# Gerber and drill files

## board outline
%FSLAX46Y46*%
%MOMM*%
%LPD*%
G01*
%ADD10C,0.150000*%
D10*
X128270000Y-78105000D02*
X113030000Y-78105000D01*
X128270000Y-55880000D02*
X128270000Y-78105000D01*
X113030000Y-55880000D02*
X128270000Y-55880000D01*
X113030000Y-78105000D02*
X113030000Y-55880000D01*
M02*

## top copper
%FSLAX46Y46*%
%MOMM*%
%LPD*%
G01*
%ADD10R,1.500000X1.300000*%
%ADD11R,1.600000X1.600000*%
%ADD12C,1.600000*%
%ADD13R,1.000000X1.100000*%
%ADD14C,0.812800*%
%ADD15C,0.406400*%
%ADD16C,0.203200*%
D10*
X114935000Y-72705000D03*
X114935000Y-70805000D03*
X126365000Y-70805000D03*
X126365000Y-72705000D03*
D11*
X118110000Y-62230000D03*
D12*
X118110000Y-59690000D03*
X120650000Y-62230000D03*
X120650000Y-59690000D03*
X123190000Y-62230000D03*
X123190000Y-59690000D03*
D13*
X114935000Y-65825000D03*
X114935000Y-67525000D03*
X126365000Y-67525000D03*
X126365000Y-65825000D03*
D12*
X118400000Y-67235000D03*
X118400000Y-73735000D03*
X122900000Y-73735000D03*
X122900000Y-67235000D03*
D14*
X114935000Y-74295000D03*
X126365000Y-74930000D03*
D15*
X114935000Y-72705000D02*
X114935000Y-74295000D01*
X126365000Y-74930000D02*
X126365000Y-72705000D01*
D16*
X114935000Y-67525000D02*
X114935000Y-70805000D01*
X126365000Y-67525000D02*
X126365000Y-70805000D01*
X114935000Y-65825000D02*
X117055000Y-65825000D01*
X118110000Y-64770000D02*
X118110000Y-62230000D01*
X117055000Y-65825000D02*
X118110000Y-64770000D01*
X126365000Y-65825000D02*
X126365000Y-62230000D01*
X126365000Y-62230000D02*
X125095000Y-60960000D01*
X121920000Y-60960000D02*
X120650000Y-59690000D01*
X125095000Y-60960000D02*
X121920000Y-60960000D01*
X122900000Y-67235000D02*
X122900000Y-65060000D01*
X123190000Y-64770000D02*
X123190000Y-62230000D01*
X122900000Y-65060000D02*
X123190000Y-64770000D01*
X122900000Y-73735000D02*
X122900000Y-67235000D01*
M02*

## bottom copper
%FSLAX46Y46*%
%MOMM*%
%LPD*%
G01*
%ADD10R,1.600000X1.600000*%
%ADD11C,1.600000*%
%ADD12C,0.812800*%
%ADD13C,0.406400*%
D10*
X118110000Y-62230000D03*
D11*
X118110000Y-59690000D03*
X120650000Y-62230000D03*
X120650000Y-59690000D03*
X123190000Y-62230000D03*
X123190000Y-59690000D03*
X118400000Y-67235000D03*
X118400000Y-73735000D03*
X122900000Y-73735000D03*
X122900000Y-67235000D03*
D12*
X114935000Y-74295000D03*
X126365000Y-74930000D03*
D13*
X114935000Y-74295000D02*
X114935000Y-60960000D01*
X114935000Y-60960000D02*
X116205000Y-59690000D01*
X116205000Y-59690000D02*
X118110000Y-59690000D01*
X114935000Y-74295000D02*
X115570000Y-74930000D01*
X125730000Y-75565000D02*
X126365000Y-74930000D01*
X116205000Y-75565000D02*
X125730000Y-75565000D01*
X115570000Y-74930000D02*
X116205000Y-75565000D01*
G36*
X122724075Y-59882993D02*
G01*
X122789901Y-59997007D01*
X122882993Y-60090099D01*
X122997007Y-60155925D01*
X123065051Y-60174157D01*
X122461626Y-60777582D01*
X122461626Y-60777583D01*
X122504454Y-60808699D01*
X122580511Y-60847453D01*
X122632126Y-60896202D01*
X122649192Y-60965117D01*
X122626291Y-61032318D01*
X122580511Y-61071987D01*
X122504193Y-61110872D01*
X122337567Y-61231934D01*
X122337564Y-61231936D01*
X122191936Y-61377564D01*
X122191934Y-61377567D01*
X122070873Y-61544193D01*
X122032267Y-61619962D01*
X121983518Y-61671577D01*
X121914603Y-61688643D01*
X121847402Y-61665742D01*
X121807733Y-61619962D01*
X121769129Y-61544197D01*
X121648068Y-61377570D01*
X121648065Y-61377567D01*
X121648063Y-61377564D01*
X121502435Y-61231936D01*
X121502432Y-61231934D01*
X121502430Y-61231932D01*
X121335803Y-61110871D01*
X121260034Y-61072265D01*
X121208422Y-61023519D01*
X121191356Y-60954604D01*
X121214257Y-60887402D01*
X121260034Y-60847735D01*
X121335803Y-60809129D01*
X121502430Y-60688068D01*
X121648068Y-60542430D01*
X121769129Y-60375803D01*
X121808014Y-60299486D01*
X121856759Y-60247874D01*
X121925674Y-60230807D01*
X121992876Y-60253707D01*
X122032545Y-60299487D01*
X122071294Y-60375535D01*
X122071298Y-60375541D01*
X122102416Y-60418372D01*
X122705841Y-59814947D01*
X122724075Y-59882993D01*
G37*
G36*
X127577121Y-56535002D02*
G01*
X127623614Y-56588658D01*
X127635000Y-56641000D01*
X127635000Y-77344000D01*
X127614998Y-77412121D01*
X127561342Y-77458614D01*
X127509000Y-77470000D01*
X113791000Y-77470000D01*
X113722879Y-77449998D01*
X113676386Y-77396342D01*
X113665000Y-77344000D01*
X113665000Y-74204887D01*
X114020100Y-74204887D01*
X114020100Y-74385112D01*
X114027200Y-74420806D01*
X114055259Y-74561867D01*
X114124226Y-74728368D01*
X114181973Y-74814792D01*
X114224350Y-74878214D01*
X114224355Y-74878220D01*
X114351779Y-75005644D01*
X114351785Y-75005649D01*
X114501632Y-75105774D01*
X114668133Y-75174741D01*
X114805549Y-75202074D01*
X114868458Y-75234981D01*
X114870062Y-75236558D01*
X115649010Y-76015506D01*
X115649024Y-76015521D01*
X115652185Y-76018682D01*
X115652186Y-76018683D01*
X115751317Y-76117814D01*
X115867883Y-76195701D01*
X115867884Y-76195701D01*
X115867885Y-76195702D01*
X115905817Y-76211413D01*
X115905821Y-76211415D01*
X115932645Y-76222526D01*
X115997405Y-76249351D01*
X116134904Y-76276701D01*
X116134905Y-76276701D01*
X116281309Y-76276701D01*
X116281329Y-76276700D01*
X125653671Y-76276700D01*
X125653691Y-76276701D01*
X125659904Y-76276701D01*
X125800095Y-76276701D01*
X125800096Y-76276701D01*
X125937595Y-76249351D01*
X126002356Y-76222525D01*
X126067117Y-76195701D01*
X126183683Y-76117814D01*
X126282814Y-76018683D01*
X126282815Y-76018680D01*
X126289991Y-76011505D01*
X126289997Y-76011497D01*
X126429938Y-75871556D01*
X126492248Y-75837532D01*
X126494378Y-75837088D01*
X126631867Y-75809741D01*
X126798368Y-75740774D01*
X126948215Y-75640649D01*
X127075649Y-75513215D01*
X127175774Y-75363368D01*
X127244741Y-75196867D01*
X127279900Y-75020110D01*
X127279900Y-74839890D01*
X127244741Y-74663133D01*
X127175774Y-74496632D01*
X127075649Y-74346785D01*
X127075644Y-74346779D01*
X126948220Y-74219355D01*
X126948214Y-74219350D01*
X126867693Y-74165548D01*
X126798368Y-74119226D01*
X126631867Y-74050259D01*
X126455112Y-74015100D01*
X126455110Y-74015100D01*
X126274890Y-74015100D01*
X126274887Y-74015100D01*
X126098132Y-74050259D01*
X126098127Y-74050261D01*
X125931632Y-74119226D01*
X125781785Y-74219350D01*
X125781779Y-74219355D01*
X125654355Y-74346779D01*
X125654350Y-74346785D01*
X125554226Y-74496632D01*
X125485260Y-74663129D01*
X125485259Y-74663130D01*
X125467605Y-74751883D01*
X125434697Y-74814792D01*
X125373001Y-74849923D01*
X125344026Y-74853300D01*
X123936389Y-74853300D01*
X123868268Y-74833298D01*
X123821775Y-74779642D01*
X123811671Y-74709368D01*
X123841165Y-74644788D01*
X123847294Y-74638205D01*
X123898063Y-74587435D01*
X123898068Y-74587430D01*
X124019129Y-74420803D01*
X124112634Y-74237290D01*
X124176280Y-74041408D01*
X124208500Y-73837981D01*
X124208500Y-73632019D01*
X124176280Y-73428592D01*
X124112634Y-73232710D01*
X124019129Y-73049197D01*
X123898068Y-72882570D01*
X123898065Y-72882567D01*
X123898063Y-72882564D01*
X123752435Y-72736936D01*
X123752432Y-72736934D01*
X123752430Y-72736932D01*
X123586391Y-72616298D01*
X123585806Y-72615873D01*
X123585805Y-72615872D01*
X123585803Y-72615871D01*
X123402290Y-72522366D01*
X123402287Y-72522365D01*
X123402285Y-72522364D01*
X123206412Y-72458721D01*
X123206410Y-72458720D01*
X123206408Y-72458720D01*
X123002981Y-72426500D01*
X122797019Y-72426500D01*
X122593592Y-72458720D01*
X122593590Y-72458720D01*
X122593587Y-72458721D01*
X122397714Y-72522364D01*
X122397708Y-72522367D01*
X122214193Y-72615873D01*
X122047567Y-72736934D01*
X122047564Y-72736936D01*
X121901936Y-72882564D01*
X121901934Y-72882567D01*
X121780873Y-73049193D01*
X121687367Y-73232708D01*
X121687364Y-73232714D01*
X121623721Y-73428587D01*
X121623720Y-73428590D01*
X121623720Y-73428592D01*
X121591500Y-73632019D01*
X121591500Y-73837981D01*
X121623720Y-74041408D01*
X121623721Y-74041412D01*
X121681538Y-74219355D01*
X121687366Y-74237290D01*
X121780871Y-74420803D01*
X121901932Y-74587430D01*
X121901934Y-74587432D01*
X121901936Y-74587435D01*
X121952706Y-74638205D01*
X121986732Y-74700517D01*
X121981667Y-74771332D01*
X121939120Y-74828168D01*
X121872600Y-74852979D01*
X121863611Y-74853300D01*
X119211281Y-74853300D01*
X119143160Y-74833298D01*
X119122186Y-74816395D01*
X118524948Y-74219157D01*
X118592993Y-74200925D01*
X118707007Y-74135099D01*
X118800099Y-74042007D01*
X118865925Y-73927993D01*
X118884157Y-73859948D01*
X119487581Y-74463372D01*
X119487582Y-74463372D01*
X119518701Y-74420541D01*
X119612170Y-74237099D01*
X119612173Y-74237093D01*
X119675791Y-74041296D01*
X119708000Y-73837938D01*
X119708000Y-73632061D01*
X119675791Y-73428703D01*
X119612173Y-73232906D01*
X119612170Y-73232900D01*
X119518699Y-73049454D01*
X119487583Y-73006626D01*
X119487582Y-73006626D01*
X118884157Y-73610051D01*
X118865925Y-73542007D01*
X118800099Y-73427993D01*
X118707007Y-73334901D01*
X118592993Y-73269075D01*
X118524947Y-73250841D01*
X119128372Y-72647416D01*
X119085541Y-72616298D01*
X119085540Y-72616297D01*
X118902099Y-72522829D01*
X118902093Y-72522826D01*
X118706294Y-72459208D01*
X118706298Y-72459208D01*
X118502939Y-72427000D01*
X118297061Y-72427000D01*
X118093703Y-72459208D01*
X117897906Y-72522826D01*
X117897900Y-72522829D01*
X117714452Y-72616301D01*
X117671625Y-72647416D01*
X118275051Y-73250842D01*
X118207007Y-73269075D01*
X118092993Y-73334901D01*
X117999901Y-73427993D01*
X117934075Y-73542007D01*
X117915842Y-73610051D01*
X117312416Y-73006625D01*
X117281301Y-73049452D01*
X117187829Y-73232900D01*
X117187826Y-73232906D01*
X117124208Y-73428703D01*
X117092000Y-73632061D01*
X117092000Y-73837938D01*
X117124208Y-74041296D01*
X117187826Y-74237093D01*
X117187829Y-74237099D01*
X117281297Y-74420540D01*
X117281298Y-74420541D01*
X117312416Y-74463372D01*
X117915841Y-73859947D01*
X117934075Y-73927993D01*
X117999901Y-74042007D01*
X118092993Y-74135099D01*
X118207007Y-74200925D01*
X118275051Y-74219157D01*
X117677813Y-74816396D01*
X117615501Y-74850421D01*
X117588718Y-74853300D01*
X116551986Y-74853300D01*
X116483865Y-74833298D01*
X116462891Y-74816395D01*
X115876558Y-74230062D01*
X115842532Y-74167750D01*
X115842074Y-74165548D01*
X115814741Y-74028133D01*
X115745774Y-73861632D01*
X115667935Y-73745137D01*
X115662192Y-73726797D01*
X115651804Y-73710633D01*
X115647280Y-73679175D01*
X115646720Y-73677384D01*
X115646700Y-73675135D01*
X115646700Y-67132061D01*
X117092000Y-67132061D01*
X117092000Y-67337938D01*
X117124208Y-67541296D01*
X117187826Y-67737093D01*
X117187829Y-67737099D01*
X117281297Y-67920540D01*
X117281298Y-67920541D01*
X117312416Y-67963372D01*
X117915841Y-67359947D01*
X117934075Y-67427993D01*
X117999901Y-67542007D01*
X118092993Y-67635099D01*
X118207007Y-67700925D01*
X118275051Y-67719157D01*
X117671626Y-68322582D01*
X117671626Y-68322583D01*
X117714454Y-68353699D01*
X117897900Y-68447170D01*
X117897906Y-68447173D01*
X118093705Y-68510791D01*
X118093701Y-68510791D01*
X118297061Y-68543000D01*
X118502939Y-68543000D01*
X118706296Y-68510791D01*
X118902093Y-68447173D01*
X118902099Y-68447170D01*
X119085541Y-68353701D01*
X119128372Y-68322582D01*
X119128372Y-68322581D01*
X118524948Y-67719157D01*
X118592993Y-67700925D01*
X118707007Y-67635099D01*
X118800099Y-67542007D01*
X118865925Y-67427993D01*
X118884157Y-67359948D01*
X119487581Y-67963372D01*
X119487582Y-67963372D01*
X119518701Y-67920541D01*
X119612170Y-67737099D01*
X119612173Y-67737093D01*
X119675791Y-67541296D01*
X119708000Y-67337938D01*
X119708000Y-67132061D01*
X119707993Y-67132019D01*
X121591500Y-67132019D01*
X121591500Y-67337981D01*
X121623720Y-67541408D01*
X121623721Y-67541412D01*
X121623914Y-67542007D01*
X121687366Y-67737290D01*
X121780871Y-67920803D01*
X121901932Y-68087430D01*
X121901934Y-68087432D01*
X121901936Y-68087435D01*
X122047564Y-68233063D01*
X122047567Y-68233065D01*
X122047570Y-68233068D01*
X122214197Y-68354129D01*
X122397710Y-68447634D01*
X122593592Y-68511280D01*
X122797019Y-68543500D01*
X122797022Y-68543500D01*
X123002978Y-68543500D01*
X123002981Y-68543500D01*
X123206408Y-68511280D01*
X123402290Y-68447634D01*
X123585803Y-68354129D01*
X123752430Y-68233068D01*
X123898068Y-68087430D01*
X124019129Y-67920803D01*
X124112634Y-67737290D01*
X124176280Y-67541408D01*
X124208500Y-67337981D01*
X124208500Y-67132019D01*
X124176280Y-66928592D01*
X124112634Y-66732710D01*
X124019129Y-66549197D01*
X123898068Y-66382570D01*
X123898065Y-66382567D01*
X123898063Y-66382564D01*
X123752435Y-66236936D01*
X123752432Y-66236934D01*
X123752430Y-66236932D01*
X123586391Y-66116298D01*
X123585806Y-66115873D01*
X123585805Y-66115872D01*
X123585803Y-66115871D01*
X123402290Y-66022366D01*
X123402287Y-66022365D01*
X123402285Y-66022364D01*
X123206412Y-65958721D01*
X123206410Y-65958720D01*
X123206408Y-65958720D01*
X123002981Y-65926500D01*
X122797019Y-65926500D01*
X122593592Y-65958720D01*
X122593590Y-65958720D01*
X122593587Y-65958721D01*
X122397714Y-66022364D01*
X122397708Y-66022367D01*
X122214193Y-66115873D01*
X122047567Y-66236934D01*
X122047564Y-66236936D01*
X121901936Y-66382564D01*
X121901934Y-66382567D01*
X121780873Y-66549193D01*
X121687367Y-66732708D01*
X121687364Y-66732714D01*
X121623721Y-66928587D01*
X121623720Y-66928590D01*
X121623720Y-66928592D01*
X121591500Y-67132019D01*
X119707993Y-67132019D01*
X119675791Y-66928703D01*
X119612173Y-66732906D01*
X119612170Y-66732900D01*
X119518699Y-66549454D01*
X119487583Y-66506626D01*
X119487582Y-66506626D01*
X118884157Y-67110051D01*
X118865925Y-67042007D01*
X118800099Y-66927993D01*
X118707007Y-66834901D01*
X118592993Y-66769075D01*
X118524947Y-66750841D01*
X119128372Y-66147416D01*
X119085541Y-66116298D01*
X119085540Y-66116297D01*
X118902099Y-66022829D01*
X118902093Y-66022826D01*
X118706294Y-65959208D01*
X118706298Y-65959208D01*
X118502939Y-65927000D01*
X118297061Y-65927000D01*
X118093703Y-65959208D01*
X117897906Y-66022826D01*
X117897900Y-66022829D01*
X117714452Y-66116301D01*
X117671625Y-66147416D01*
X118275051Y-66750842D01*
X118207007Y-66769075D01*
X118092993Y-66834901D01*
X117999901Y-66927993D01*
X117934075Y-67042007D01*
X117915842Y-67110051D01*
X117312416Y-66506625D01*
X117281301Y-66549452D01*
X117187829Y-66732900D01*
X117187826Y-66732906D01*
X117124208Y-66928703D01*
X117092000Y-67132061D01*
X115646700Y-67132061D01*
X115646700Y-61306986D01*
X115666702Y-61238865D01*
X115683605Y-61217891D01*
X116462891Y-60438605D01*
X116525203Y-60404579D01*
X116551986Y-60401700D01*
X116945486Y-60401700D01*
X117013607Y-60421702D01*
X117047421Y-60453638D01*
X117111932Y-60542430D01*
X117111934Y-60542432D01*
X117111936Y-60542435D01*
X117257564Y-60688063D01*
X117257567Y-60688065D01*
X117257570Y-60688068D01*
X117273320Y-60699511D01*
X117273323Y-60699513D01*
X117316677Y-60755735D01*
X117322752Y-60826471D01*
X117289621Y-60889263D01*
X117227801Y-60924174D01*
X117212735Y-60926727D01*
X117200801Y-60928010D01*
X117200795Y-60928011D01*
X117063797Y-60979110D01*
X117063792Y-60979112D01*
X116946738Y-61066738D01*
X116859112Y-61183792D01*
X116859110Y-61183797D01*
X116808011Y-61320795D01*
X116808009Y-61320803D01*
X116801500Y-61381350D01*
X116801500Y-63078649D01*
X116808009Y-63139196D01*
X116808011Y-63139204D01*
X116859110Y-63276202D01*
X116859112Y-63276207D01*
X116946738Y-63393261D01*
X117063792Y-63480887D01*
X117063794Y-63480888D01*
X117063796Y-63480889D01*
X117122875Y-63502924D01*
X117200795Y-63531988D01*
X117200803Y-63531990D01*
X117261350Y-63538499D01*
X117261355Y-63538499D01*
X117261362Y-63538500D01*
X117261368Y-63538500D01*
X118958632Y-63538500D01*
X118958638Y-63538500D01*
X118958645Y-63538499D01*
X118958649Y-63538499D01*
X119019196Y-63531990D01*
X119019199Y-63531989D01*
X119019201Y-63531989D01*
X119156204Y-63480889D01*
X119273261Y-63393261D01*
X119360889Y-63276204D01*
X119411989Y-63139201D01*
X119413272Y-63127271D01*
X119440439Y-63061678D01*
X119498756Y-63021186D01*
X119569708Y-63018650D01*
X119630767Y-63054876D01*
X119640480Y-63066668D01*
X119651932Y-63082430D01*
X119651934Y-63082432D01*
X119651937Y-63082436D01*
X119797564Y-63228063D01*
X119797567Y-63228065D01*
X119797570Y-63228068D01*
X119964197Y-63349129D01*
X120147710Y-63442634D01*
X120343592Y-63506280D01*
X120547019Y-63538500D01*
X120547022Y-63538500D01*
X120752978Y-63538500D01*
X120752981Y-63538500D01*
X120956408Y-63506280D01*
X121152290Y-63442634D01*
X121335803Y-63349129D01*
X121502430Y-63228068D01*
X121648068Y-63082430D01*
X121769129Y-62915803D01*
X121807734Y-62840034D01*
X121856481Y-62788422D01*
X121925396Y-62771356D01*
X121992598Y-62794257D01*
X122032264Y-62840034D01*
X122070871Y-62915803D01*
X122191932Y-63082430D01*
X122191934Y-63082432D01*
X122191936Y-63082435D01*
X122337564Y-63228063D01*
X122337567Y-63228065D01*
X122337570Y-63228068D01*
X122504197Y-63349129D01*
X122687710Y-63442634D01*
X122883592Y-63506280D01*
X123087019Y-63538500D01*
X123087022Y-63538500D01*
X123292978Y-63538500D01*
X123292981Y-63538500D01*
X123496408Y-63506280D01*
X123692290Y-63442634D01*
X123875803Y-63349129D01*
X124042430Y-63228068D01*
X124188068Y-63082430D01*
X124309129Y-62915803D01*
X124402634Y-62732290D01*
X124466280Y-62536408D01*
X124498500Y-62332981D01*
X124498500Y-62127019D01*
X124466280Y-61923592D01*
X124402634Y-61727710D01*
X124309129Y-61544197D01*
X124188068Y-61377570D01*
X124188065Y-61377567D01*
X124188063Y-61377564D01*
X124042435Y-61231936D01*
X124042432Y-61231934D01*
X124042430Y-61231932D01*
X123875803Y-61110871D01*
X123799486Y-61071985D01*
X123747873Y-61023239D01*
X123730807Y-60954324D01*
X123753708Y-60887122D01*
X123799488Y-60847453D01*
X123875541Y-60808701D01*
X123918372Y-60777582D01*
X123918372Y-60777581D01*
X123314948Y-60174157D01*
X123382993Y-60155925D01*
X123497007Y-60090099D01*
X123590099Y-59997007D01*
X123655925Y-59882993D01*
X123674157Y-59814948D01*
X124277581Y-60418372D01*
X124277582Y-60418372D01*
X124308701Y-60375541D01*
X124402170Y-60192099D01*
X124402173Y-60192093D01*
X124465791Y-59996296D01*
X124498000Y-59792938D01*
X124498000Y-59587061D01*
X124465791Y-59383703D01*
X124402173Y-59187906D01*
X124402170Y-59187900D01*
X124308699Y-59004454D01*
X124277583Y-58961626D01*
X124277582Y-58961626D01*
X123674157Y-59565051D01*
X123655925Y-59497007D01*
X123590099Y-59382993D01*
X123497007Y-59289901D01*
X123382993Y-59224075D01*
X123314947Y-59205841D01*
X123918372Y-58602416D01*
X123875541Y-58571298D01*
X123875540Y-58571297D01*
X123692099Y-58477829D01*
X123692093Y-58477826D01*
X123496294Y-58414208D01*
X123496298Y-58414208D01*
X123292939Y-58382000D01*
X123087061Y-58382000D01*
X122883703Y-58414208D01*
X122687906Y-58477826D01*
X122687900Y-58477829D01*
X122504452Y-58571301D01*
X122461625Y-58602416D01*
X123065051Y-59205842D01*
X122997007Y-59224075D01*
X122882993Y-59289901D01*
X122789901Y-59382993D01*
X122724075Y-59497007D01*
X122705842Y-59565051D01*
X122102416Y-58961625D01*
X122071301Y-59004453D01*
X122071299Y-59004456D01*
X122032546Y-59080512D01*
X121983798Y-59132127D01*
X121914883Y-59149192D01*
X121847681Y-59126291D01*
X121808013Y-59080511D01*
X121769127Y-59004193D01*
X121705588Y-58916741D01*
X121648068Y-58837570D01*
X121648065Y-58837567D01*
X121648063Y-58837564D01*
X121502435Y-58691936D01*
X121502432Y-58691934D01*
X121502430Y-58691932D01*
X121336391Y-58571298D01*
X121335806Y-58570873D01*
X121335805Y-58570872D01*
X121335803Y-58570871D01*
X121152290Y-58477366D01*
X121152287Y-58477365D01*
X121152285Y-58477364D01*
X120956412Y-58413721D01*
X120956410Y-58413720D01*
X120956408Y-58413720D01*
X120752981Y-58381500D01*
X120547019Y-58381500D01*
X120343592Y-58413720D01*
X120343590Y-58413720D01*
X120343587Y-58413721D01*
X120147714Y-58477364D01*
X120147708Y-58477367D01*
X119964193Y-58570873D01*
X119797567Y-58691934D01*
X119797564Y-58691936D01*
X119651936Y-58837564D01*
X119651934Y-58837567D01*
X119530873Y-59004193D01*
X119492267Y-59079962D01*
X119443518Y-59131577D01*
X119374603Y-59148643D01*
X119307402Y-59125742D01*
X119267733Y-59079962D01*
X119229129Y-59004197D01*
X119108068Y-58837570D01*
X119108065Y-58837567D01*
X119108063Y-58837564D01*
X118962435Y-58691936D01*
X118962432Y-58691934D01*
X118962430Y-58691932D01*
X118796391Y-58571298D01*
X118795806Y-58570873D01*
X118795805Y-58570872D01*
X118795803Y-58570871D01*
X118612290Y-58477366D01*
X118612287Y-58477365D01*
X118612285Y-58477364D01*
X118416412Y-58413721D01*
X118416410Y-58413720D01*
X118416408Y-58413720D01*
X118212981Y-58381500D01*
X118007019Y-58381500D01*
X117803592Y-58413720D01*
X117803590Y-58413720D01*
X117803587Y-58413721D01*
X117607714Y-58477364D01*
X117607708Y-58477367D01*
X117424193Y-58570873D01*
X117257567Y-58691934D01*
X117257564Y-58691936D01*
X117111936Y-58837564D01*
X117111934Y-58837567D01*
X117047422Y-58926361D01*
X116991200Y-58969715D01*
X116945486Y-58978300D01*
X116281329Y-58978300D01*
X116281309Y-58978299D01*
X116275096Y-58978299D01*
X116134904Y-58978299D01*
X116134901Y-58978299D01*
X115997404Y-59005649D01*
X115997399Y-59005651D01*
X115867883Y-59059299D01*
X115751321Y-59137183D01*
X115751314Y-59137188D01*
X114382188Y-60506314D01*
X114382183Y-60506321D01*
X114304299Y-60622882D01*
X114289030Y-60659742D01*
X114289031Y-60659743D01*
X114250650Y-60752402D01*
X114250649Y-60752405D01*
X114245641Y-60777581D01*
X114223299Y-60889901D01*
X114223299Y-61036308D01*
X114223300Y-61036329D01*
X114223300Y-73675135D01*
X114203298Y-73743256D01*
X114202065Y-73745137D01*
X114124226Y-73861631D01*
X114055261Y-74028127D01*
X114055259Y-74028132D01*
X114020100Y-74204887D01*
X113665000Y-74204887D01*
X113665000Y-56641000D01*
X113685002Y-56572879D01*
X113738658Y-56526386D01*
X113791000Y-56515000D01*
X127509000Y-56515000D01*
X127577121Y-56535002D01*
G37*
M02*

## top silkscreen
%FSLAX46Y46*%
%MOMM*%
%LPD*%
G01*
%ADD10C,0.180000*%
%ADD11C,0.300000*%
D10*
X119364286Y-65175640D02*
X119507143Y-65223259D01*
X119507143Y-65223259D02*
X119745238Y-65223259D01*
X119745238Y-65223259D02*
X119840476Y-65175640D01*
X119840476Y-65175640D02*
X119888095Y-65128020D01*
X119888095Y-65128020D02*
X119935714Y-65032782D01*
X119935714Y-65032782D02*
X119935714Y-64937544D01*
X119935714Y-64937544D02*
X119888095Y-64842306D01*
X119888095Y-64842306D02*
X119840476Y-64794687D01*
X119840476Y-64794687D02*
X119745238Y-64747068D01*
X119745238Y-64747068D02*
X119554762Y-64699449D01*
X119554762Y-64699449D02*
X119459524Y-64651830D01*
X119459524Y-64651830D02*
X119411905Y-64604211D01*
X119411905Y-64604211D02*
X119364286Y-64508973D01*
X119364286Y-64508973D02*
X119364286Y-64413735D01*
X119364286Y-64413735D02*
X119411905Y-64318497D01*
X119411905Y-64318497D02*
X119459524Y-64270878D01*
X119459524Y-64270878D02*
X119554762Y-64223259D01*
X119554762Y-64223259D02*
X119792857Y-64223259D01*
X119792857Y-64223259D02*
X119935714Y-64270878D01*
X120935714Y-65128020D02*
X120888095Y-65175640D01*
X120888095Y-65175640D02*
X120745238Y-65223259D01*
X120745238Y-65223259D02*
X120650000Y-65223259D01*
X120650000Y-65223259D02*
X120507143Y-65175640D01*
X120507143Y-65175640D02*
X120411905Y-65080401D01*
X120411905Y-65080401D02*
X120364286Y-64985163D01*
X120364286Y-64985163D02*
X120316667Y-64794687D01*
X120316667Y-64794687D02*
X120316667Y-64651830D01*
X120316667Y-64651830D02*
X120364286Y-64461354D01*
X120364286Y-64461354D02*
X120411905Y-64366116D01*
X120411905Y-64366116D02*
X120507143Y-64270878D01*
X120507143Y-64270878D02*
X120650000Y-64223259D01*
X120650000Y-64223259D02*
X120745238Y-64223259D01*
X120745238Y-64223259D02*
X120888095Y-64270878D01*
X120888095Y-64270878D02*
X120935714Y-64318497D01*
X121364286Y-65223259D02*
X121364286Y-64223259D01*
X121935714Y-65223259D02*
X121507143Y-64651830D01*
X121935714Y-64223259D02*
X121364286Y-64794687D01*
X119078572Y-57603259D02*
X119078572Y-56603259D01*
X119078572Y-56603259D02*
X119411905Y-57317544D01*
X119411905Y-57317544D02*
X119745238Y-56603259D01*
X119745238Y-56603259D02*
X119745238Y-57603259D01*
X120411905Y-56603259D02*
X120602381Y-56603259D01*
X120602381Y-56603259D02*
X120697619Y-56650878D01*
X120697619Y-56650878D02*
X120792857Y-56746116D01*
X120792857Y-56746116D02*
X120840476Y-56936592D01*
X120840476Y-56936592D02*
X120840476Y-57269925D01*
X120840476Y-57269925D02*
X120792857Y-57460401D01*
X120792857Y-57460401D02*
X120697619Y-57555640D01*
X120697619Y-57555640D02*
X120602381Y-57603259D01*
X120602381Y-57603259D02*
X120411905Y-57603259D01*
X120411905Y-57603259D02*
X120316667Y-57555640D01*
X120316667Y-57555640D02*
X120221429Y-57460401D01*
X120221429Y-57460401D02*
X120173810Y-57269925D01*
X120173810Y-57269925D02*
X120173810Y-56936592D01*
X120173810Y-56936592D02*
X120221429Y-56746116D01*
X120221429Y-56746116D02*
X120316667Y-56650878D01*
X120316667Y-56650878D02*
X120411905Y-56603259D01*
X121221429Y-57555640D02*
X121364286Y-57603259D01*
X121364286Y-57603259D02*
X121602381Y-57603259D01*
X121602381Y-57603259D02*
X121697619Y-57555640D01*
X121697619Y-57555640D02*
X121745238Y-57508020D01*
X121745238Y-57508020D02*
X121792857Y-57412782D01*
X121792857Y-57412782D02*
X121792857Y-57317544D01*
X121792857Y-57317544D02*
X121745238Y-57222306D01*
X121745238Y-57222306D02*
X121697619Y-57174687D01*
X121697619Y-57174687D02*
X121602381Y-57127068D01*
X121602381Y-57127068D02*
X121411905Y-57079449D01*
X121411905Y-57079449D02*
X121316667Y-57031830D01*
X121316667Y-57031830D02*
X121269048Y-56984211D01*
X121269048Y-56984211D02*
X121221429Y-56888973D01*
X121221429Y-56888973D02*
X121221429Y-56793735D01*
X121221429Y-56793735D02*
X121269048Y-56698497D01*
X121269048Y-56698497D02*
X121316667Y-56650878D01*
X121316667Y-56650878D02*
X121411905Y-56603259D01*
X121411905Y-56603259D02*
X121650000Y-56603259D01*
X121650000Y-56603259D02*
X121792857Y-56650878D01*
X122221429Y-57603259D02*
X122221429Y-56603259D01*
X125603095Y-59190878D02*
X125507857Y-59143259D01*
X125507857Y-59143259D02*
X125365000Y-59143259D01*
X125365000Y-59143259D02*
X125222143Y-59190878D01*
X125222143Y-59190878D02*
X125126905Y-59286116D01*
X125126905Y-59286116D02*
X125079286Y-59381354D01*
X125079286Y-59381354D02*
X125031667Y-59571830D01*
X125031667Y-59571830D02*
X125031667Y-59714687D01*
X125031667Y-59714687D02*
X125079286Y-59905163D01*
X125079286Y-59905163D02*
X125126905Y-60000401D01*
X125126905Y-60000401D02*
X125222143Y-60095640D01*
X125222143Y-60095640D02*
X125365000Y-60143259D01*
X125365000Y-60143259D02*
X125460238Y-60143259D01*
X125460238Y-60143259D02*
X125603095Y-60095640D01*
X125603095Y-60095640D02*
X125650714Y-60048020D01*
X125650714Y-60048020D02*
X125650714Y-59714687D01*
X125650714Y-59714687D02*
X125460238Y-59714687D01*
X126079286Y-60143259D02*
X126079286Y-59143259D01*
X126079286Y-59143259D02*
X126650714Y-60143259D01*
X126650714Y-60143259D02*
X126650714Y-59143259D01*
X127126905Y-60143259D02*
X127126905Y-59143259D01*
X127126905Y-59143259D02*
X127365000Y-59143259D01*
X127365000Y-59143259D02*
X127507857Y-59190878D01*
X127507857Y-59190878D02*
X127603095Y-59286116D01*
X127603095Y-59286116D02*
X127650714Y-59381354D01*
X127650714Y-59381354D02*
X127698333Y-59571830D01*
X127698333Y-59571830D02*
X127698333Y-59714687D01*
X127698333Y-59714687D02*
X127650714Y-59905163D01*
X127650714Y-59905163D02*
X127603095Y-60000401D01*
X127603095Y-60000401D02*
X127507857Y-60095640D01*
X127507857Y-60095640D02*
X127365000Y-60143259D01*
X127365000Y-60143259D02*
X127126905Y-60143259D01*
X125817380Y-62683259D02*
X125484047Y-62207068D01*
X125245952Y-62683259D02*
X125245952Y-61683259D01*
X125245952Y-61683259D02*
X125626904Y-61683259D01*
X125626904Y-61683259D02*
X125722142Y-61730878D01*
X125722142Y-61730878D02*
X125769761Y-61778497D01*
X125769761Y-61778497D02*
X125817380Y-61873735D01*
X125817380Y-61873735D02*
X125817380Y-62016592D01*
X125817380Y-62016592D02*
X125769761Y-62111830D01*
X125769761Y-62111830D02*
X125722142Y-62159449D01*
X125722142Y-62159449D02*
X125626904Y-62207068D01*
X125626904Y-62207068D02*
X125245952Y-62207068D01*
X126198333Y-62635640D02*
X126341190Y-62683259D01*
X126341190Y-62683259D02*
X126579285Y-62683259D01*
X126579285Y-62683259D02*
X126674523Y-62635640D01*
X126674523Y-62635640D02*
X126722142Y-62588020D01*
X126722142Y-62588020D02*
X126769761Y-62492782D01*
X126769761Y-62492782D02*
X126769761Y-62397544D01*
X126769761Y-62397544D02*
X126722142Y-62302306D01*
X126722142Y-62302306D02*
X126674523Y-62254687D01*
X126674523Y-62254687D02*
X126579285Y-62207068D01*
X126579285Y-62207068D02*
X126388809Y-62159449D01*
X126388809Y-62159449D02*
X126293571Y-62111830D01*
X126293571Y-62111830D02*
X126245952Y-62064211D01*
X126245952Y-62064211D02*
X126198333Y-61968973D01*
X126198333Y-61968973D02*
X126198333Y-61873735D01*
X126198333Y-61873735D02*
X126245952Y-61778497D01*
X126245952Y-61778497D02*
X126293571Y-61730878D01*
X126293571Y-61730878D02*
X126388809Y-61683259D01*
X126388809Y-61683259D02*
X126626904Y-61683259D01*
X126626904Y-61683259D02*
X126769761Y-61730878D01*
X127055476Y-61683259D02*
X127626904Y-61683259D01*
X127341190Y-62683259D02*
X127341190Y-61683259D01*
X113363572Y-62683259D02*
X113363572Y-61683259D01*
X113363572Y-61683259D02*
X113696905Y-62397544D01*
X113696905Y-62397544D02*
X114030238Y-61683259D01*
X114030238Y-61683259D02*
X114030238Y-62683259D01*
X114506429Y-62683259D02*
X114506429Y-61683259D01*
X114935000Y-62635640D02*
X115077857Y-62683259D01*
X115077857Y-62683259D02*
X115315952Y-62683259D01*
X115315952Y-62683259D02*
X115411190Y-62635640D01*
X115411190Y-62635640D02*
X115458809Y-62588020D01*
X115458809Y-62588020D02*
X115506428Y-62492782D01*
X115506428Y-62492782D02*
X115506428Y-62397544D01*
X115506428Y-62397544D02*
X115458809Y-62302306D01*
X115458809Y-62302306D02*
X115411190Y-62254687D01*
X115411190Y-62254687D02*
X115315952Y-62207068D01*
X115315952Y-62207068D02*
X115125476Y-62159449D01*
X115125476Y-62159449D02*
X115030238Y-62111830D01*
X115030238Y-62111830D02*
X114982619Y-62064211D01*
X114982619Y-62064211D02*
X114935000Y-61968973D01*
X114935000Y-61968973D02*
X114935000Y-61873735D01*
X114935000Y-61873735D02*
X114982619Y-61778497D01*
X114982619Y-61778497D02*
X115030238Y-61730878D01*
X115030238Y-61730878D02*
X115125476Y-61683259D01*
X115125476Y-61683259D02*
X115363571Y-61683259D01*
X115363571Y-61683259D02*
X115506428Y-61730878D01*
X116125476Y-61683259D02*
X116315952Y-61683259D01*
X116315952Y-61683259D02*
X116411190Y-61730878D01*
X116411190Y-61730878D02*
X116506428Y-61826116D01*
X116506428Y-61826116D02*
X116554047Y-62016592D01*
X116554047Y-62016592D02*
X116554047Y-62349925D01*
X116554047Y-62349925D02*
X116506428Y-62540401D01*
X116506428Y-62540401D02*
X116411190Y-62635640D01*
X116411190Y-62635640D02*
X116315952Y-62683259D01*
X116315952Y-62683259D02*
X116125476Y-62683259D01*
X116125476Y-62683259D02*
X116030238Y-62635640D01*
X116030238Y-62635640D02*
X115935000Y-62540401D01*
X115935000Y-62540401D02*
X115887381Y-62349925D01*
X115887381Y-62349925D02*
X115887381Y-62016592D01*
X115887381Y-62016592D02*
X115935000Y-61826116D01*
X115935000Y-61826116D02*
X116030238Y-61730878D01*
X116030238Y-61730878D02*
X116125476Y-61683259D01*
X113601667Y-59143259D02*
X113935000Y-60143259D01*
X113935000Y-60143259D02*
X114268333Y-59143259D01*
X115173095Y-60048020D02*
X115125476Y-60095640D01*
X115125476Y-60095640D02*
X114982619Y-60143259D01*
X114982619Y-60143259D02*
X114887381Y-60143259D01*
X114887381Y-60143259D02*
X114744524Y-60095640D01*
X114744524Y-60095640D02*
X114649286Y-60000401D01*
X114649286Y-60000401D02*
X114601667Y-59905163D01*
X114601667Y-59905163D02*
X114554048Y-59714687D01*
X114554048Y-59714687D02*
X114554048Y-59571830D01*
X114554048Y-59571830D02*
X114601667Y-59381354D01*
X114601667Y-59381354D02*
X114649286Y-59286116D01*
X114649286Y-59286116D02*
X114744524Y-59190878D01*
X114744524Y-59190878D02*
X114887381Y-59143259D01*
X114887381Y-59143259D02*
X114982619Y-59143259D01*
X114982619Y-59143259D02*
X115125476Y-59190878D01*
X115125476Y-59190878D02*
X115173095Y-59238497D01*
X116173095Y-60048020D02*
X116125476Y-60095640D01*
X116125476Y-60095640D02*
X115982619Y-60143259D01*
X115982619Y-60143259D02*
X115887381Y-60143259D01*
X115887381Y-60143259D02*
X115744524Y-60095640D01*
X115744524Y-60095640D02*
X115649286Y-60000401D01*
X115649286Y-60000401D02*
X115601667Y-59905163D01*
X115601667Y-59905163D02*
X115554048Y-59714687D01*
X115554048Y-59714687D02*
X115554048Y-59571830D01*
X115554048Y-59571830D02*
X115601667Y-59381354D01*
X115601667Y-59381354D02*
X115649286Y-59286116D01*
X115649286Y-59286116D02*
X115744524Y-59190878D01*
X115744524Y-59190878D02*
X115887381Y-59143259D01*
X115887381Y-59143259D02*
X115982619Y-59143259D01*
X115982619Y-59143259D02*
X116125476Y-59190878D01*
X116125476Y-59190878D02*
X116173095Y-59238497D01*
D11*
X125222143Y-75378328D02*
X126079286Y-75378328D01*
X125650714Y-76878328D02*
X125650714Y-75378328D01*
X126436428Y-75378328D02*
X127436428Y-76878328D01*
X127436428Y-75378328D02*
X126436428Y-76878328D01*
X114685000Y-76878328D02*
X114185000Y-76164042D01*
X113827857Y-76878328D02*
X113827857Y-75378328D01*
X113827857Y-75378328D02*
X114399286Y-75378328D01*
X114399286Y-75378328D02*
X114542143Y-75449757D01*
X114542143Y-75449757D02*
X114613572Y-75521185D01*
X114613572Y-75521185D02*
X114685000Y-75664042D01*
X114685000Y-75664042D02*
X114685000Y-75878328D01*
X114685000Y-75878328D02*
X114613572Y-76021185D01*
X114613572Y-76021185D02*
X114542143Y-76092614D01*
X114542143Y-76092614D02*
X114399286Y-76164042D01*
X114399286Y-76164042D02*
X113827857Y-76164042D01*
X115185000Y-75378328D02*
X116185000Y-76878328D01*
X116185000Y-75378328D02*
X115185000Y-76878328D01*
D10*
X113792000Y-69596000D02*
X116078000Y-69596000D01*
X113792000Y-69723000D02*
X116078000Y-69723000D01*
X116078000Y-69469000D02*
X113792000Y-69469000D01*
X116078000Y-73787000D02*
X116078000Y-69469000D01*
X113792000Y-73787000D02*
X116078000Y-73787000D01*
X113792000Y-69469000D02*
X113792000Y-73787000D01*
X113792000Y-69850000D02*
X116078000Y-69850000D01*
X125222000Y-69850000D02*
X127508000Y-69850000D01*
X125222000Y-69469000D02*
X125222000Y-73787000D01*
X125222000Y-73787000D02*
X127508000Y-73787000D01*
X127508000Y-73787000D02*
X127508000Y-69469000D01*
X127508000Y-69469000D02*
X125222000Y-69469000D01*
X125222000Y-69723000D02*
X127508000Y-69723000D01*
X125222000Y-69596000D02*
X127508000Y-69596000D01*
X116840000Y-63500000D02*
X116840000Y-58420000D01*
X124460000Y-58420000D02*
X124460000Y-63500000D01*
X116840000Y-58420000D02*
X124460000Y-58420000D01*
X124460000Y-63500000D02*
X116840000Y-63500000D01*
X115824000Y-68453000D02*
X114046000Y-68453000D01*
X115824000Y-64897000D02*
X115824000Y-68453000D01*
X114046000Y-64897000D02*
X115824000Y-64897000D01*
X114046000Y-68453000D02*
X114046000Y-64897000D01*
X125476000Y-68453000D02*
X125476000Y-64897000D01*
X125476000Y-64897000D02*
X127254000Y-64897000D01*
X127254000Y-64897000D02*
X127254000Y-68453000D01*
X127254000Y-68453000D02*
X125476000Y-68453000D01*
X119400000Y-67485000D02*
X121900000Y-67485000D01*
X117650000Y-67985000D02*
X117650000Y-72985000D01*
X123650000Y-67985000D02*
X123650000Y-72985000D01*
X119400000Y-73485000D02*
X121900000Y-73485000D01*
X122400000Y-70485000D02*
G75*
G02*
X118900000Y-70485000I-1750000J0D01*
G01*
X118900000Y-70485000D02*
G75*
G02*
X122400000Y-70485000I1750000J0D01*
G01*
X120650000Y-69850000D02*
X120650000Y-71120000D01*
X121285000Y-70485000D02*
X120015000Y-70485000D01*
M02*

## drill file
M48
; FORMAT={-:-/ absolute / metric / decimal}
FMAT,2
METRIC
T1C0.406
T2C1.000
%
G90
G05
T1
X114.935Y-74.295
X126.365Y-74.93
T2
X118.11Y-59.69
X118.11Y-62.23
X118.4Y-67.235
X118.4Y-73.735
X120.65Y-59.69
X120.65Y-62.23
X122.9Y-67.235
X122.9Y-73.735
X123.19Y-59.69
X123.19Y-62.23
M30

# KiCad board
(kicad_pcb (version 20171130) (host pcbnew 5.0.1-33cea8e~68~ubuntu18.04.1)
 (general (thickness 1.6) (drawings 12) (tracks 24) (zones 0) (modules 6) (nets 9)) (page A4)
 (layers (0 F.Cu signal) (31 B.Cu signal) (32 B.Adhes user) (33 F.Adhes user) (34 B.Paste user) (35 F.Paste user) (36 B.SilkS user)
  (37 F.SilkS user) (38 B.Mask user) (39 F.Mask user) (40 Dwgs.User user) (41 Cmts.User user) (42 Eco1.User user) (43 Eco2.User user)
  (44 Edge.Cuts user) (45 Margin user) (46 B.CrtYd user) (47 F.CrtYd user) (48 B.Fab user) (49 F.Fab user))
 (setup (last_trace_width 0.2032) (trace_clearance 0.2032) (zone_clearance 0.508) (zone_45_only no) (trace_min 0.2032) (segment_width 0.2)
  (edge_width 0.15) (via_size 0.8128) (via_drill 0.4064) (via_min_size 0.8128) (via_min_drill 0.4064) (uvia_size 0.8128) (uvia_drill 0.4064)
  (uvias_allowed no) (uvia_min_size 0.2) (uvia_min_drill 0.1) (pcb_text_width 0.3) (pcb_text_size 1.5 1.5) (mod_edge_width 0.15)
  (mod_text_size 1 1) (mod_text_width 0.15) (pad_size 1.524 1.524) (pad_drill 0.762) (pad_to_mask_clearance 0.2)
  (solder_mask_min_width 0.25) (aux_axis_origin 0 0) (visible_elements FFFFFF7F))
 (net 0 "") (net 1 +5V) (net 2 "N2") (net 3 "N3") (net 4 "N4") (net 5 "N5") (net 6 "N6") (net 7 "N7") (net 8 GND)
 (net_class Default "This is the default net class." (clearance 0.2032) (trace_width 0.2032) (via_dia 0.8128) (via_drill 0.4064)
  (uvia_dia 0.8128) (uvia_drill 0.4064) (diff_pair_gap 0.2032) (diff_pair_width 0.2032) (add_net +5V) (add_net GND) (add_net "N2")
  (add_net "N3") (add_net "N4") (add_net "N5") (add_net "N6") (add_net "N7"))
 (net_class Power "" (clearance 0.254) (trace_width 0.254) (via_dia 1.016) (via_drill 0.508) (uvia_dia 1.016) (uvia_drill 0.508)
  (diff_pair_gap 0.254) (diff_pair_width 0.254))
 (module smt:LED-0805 (layer F.Cu) (at 114.935 71.755 270)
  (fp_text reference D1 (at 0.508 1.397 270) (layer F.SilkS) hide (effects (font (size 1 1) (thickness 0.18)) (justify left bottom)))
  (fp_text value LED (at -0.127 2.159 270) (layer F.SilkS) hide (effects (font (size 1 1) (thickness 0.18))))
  (fp_line (start -2.159 1.143) (end -2.159 -1.143) (layer F.SilkS) (width 0.18))
  (fp_line (start -2.032 1.143) (end -2.032 -1.143) (layer F.SilkS) (width 0.18))
  (fp_line (start -2.286 -1.143) (end -2.286 1.143) (layer F.SilkS) (width 0.18))
  (fp_line (start 2.032 -1.143) (end -2.286 -1.143) (layer F.SilkS) (width 0.18))
  (fp_line (start 2.032 1.143) (end 2.032 -1.143) (layer F.SilkS) (width 0.18))
  (fp_line (start -2.286 1.143) (end 2.032 1.143) (layer F.SilkS) (width 0.18))
  (fp_line (start -1.905 1.143) (end -1.905 -1.143) (layer F.SilkS) (width 0.18))
  (pad A smd rect (at 0.95 0 270) (size 1.3 1.5) (layers F.Cu F.Paste F.Mask) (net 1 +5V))
  (pad K smd rect (at -0.95 0 270) (size 1.3 1.5) (layers F.Cu F.Paste F.Mask) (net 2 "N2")))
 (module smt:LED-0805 (layer F.Cu) (at 126.365 71.755 270)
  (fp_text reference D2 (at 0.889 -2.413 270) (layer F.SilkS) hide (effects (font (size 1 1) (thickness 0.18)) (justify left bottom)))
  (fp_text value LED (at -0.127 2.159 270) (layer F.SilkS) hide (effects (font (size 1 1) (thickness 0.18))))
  (fp_line (start -1.905 1.143) (end -1.905 -1.143) (layer F.SilkS) (width 0.18))
  (fp_line (start -2.286 1.143) (end 2.032 1.143) (layer F.SilkS) (width 0.18))
  (fp_line (start 2.032 1.143) (end 2.032 -1.143) (layer F.SilkS) (width 0.18))
  (fp_line (start 2.032 -1.143) (end -2.286 -1.143) (layer F.SilkS) (width 0.18))
  (fp_line (start -2.286 -1.143) (end -2.286 1.143) (layer F.SilkS) (width 0.18))
  (fp_line (start -2.032 1.143) (end -2.032 -1.143) (layer F.SilkS) (width 0.18))
  (fp_line (start -2.159 1.143) (end -2.159 -1.143) (layer F.SilkS) (width 0.18))
  (pad K smd rect (at -0.95 0 270) (size 1.3 1.5) (layers F.Cu F.Paste F.Mask) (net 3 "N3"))
  (pad A smd rect (at 0.95 0 270) (size 1.3 1.5) (layers F.Cu F.Paste F.Mask) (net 1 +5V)))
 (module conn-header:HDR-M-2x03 (layer F.Cu) (at 120.65 60.96)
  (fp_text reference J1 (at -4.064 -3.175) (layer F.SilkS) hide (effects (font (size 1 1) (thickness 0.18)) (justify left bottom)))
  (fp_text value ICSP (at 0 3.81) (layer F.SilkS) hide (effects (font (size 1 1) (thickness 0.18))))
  (fp_line (start -3.81 2.54) (end -3.81 -2.54) (layer F.SilkS) (width 0.18))
  (fp_line (start 3.81 -2.54) (end 3.81 2.54) (layer F.SilkS) (width 0.18))
  (fp_line (start -3.81 -2.54) (end 3.81 -2.54) (layer F.SilkS) (width 0.18))
  (fp_line (start 3.81 2.54) (end -3.81 2.54) (layer F.SilkS) (width 0.18))
  (pad 1 thru_hole rect (at -2.54 1.27) (size 1.6 1.6) (drill 1) (layers *.Cu *.Mask) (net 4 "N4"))
  (pad 2 thru_hole circle (at -2.54 -1.27) (size 1.6 1.6) (drill 1) (layers *.Cu *.Mask) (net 1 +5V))
  (pad 3 thru_hole circle (at 0 1.27) (size 1.6 1.6) (drill 1) (layers *.Cu *.Mask) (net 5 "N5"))
  (pad 4 thru_hole circle (at 0 -1.27) (size 1.6 1.6) (drill 1) (layers *.Cu *.Mask) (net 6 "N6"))
  (pad 5 thru_hole circle (at 2.54 1.27) (size 1.6 1.6) (drill 1) (layers *.Cu *.Mask) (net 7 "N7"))
  (pad 6 thru_hole circle (at 2.54 -1.27) (size 1.6 1.6) (drill 1) (layers *.Cu *.Mask) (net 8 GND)))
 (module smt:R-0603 (layer F.Cu) (at 114.935 66.675 90)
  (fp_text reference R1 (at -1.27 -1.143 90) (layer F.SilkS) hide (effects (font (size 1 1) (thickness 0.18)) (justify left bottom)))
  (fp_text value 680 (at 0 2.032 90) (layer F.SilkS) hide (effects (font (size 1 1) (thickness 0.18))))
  (fp_line (start -1.778 0.889) (end -1.778 -0.889) (layer F.SilkS) (width 0.18))
  (fp_line (start 1.778 0.889) (end -1.778 0.889) (layer F.SilkS) (width 0.18))
  (fp_line (start 1.778 -0.889) (end 1.778 0.889) (layer F.SilkS) (width 0.18))
  (fp_line (start -1.778 -0.889) (end 1.778 -0.889) (layer F.SilkS) (width 0.18))
  (pad 2 smd rect (at 0.85 0 90) (size 1.1 1) (layers F.Cu F.Paste F.Mask) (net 4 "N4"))
  (pad 1 smd rect (at -0.85 0 90) (size 1.1 1) (layers F.Cu F.Paste F.Mask) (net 2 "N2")))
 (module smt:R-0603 (layer F.Cu) (at 126.365 66.675 90)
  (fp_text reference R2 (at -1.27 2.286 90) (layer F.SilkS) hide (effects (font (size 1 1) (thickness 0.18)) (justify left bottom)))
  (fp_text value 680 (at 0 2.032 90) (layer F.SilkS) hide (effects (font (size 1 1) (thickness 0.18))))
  (fp_line (start -1.778 -0.889) (end 1.778 -0.889) (layer F.SilkS) (width 0.18))
  (fp_line (start 1.778 -0.889) (end 1.778 0.889) (layer F.SilkS) (width 0.18))
  (fp_line (start 1.778 0.889) (end -1.778 0.889) (layer F.SilkS) (width 0.18))
  (fp_line (start -1.778 0.889) (end -1.778 -0.889) (layer F.SilkS) (width 0.18))
  (pad 1 smd rect (at -0.85 0 90) (size 1.1 1) (layers F.Cu F.Paste F.Mask) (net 3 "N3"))
  (pad 2 smd rect (at 0.85 0 90) (size 1.1 1) (layers F.Cu F.Paste F.Mask) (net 6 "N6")))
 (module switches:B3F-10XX (layer F.Cu) (at 120.65 70.485 270)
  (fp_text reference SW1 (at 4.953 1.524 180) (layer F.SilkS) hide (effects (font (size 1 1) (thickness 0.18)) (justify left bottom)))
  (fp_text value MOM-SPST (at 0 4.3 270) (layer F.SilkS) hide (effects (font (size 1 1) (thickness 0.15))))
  (fp_line (start -3 1.25) (end -3 -1.25) (layer F.SilkS) (width 0.18))
  (fp_line (start -2.5 3) (end 2.5 3) (layer F.SilkS) (width 0.18))
  (fp_line (start -2.5 -3) (end 2.5 -3) (layer F.SilkS) (width 0.18))
  (fp_line (start 3 1.25) (end 3 -1.25) (layer F.SilkS) (width 0.18))
  (fp_circle (center 0 0) (end 1.75 0) (layer F.SilkS) (width 0.18))
  (fp_line (start -0.635 0) (end 0.635 0) (layer F.SilkS) (width 0.18))
  (fp_line (start 0 -0.635) (end 0 0.635) (layer F.SilkS) (width 0.18))
  (pad 1 thru_hole circle (at -3.25 2.25 270) (size 1.6 1.6) (drill 1) (layers *.Cu *.Mask) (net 8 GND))
  (pad 1 thru_hole circle (at 3.25 2.25 270) (size 1.6 1.6) (drill 1) (layers *.Cu *.Mask) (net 8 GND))
  (pad 2 thru_hole circle (at 3.25 -2.25 270) (size 1.6 1.6) (drill 1) (layers *.Cu *.Mask) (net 7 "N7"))
  (pad 2 thru_hole circle (at -3.25 -2.25 270) (size 1.6 1.6) (drill 1) (layers *.Cu *.Mask) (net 7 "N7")))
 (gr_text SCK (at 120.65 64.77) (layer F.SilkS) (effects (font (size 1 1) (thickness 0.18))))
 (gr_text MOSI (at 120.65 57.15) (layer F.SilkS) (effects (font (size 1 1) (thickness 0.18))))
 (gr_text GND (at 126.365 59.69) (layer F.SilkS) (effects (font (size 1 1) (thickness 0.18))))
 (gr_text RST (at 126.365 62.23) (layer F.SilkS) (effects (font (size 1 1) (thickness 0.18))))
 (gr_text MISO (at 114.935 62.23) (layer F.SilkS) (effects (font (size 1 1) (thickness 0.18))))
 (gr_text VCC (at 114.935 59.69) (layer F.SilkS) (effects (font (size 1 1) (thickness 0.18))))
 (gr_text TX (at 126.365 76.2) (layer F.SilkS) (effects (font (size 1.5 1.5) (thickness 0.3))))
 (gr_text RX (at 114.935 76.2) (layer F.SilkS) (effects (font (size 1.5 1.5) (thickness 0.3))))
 (gr_line (start 128.27 78.105) (end 113.03 78.105) (layer Edge.Cuts) (width 0.15))
 (gr_line (start 128.27 55.88) (end 128.27 78.105) (layer Edge.Cuts) (width 0.15))
 (gr_line (start 113.03 55.88) (end 128.27 55.88) (layer Edge.Cuts) (width 0.15))
 (gr_line (start 113.03 78.105) (end 113.03 55.88) (layer Edge.Cuts) (width 0.15))
 (via (at 114.935 74.295) (size 0.8128) (drill 0.4064) (layers F.Cu B.Cu) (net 1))
 (segment (start 114.935 72.705) (end 114.935 74.295) (width 0.4064) (layer F.Cu) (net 1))
 (segment (start 114.935 74.295) (end 114.935 60.96) (width 0.4064) (layer B.Cu) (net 1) (status 1000000))
 (segment (start 114.935 60.96) (end 116.205 59.69) (width 0.4064) (layer B.Cu) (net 1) (status 1000000))
 (segment (start 116.205 59.69) (end 118.11 59.69) (width 0.4064) (layer B.Cu) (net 1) (status 1000000))
 (segment (start 114.935 74.295) (end 115.57 74.93) (width 0.4064) (layer B.Cu) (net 1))
 (segment (start 126.365 74.93) (end 126.365 72.705) (width 0.4064) (layer F.Cu) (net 1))
 (segment (start 125.73 75.565) (end 126.365 74.93) (width 0.4064) (layer B.Cu) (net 1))
 (segment (start 116.205 75.565) (end 125.73 75.565) (width 0.4064) (layer B.Cu) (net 1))
 (via (at 126.365 74.93) (size 0.8128) (drill 0.4064) (layers F.Cu B.Cu) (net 1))
 (segment (start 115.57 74.93) (end 116.205 75.565) (width 0.4064) (layer B.Cu) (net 1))
 (segment (start 114.935 67.525) (end 114.935 70.805) (width 0.2032) (layer F.Cu) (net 2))
 (segment (start 126.365 67.525) (end 126.365 70.805) (width 0.2032) (layer F.Cu) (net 3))
 (segment (start 114.935 65.825) (end 117.055 65.825) (width 0.2032) (layer F.Cu) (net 4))
 (segment (start 118.11 64.77) (end 118.11 62.23) (width 0.2032) (layer F.Cu) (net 4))
 (segment (start 117.055 65.825) (end 118.11 64.77) (width 0.2032) (layer F.Cu) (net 4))
 (segment (start 126.365 65.825) (end 126.365 62.23) (width 0.2032) (layer F.Cu) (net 6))
 (segment (start 126.365 62.23) (end 125.095 60.96) (width 0.2032) (layer F.Cu) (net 6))
 (segment (start 121.92 60.96) (end 120.65 59.69) (width 0.2032) (layer F.Cu) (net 6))
 (segment (start 125.095 60.96) (end 121.92 60.96) (width 0.2032) (layer F.Cu) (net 6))
 (segment (start 122.9 67.235) (end 122.9 65.06) (width 0.2032) (layer F.Cu) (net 7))
 (segment (start 123.19 64.77) (end 123.19 62.23) (width 0.2032) (layer F.Cu) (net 7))
 (segment (start 122.9 65.06) (end 123.19 64.77) (width 0.2032) (layer F.Cu) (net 7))
 (segment (start 122.9 73.735) (end 122.9 67.235) (width 0.2032) (layer F.Cu) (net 7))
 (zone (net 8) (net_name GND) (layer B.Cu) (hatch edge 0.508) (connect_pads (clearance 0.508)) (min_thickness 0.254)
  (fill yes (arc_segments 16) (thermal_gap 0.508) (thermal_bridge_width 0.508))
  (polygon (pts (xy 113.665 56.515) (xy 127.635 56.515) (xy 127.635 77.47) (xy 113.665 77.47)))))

